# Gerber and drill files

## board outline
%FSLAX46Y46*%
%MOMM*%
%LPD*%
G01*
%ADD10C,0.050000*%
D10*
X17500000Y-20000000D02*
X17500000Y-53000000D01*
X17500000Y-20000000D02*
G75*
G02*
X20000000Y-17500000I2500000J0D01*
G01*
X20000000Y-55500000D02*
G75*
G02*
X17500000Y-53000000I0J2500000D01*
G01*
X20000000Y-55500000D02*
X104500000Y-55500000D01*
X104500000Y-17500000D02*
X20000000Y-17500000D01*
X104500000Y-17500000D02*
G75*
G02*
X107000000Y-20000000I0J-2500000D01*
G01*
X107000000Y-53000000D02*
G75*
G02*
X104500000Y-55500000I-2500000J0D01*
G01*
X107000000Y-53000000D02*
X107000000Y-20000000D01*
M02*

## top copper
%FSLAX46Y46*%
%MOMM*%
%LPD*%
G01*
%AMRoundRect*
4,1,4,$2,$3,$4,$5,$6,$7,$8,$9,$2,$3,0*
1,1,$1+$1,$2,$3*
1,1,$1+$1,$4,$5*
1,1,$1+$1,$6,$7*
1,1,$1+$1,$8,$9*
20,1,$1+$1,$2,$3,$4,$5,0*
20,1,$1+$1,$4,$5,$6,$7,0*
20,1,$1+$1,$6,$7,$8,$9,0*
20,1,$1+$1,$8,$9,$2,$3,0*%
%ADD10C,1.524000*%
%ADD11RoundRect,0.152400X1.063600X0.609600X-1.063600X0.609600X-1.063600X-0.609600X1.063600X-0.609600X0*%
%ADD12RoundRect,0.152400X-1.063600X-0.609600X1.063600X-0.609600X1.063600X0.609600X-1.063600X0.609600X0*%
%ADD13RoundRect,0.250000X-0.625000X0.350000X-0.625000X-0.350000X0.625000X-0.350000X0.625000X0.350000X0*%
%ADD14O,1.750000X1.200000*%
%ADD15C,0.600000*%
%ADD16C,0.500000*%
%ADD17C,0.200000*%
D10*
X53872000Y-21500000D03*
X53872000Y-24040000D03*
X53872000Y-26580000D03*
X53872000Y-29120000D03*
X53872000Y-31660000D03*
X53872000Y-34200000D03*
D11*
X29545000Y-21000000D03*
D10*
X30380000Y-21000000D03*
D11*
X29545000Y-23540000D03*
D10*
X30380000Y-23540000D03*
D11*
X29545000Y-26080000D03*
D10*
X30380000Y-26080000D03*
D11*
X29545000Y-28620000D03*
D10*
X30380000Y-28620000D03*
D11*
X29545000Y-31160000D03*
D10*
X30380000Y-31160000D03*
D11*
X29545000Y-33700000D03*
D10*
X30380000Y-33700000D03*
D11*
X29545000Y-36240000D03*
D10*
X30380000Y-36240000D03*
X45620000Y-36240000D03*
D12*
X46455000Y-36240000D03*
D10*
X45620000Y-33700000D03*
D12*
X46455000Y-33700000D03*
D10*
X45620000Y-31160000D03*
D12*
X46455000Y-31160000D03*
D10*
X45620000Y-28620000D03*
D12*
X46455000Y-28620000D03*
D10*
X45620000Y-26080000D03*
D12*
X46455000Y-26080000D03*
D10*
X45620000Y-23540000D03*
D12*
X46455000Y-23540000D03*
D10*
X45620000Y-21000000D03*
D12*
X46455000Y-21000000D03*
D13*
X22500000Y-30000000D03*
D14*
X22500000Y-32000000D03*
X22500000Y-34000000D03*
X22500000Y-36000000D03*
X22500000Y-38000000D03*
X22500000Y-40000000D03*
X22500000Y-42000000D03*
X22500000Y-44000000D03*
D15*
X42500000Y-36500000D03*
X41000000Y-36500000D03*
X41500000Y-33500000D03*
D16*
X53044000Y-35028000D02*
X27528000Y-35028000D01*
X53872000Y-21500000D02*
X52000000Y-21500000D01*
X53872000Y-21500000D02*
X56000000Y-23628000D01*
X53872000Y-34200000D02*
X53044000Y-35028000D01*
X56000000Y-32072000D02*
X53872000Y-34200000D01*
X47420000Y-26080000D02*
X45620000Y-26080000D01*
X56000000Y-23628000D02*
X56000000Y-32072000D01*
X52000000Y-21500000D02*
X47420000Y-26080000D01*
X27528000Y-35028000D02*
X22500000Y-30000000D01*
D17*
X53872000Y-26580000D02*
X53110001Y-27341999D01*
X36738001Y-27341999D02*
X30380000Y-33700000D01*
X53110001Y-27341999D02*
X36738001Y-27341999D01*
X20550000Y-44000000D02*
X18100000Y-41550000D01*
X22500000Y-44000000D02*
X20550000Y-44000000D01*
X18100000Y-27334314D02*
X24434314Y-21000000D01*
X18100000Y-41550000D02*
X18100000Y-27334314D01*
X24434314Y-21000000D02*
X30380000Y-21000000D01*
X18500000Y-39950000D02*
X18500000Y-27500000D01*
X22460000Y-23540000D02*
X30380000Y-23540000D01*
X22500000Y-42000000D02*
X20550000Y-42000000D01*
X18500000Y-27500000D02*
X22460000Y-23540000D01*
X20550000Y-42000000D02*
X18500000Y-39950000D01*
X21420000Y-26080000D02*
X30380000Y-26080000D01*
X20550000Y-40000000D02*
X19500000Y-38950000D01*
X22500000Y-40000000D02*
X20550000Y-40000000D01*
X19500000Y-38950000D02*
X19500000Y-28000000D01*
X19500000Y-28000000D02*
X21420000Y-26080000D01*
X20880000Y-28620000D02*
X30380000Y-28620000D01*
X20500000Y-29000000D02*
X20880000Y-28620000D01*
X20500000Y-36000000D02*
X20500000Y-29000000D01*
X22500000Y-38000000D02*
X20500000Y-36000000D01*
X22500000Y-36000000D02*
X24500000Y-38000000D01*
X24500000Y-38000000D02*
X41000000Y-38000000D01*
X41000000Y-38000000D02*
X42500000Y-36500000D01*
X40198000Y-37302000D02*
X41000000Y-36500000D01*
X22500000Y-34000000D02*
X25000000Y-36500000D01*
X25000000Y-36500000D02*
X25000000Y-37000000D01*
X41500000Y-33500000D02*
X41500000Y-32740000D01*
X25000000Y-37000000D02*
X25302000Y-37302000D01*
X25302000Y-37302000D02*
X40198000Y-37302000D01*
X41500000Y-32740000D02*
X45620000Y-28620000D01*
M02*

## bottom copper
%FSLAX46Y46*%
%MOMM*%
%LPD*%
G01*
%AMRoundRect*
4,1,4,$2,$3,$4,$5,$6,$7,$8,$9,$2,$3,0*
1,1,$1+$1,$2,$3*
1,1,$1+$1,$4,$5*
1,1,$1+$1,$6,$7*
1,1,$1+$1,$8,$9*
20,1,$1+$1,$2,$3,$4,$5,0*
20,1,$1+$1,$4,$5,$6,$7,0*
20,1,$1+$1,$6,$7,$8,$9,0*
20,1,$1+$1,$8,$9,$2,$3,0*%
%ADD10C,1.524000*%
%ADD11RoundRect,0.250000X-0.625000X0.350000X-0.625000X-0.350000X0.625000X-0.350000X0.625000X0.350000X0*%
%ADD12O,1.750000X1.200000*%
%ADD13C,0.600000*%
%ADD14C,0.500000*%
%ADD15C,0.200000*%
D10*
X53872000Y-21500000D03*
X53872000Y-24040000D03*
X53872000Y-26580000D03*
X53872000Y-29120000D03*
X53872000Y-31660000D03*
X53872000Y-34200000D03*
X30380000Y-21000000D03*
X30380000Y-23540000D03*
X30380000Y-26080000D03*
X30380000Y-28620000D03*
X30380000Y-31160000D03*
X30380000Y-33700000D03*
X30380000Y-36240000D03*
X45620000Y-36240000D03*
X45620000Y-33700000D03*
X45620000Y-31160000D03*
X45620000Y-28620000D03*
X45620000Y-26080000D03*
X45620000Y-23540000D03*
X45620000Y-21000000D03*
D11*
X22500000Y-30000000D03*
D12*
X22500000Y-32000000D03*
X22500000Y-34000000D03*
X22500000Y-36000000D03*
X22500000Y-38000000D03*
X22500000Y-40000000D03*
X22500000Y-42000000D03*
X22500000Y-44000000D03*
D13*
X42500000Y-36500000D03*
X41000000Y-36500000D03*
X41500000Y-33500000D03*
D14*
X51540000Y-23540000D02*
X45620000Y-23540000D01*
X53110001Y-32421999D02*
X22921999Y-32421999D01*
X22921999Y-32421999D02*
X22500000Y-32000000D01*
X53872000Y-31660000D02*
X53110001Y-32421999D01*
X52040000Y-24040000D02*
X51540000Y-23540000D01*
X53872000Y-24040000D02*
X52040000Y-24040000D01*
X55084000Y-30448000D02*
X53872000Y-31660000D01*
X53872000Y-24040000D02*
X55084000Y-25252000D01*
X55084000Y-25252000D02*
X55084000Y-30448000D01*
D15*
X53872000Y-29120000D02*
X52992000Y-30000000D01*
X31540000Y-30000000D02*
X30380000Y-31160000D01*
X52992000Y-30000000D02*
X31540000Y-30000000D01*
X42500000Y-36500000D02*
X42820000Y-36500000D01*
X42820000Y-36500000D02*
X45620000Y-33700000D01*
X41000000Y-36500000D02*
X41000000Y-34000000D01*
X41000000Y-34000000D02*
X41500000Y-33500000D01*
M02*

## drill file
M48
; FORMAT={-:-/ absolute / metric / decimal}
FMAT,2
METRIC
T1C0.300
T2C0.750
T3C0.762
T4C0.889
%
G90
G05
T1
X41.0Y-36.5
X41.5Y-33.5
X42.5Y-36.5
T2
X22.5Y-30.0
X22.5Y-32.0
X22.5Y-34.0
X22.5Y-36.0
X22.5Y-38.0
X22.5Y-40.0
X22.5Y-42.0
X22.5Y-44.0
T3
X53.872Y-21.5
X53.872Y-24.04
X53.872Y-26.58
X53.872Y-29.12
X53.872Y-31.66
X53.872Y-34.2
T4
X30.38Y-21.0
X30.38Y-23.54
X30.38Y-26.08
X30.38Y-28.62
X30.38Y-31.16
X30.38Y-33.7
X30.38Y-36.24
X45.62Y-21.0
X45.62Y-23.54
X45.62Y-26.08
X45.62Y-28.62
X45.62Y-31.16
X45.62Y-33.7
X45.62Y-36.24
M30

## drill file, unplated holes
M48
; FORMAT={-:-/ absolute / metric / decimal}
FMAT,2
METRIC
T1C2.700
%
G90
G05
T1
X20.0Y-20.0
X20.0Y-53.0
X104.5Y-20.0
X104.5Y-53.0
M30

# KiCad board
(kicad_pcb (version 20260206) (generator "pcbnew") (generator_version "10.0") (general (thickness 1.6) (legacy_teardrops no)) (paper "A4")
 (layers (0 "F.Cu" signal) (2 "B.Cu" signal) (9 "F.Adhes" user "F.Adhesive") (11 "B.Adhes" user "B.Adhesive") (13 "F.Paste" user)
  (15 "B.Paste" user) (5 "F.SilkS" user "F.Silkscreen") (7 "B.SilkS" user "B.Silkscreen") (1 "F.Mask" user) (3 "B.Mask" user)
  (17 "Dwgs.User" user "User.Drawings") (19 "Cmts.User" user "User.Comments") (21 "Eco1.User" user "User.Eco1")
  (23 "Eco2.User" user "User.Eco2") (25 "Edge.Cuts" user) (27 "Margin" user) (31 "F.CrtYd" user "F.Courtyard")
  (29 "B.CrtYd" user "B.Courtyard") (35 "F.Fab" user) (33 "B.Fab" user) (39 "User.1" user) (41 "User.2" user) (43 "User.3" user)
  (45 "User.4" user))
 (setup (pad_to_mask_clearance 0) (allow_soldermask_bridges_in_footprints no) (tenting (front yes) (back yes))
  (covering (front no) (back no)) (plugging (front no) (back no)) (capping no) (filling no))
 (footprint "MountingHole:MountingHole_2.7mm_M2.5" (layer "F.Cu") (at 104.5 53)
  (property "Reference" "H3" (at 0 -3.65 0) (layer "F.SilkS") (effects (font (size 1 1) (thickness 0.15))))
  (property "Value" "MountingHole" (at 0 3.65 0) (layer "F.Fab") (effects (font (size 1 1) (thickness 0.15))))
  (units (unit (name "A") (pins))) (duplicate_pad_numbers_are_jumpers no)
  (pad "" np_thru_hole circle (at 0 0) (size 2.7 2.7) (drill 2.7) (layers "*.Cu" "*.Mask")))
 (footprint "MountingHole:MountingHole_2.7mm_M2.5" (layer "F.Cu") (at 20 20)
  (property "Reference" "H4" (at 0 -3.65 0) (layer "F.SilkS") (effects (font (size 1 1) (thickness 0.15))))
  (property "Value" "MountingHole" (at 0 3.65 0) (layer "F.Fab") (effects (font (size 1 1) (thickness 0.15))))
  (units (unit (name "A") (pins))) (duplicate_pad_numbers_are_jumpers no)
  (pad "" np_thru_hole circle (at 0 0) (size 2.7 2.7) (drill 2.7) (layers "*.Cu" "*.Mask")))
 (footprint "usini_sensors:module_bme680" (layer "F.Cu") (at 53.872 34.2)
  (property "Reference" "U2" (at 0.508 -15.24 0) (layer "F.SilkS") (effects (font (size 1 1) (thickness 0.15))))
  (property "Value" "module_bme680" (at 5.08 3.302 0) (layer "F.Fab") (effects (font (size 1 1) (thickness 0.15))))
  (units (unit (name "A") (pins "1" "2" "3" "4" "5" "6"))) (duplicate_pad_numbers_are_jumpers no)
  (pad "1" thru_hole circle (at 0 -12.7) (size 1.524 1.524) (drill 0.762) (layers "*.Cu" "*.Mask") (remove_unused_layers no) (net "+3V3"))
  (pad "2" thru_hole circle (at 0 -10.16) (size 1.524 1.524) (drill 0.762) (layers "*.Cu" "*.Mask") (remove_unused_layers no) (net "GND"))
  (pad "3" thru_hole circle (at 0 -7.62) (size 1.524 1.524) (drill 0.762) (layers "*.Cu" "*.Mask") (remove_unused_layers no) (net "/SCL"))
  (pad "4" thru_hole circle (at 0 -5.08) (size 1.524 1.524) (drill 0.762) (layers "*.Cu" "*.Mask") (remove_unused_layers no) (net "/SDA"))
  (pad "5" thru_hole circle (at 0 -2.54) (size 1.524 1.524) (drill 0.762) (layers "*.Cu" "*.Mask") (remove_unused_layers no) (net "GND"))
  (pad "6" thru_hole circle (at 0 0) (size 1.524 1.524) (drill 0.762) (layers "*.Cu" "*.Mask") (remove_unused_layers no) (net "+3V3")))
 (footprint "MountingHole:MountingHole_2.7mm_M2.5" (layer "F.Cu") (at 104.5 20)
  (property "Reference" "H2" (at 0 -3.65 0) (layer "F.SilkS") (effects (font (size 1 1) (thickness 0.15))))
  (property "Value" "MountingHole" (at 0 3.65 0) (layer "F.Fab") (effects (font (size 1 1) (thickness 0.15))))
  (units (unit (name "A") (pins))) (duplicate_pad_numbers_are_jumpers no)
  (pad "" np_thru_hole circle (at 0 0) (size 2.7 2.7) (drill 2.7) (layers "*.Cu" "*.Mask")))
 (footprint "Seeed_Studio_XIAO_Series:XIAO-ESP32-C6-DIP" (layer "F.Cu") (at 38 28.62 90)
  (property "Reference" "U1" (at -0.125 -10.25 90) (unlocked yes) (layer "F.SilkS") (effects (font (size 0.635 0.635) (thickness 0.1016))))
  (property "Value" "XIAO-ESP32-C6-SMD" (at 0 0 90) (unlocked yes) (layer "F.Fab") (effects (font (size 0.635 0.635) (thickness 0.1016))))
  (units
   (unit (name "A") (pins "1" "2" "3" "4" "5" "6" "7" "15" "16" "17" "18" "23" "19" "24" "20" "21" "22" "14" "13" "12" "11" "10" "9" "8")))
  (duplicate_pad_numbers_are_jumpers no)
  (pad "1" smd roundrect (at 7.62 -8.455 180) (size 2.432 1.524) (layers "F.Cu" "F.Mask") (roundrect_rratio 0.1) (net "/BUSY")
   (thermal_bridge_angle 45))
  (pad "1" thru_hole circle (at 7.62 -7.62 180) (size 1.524 1.524) (drill 0.889) (layers "*.Cu" "*.Mask") (remove_unused_layers no)
   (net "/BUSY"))
  (pad "2" smd roundrect (at 5.08 -8.455 180) (size 2.432 1.524) (layers "F.Cu" "F.Mask") (roundrect_rratio 0.1) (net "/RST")
   (thermal_bridge_angle 45))
  (pad "2" thru_hole circle (at 5.08 -7.62 180) (size 1.524 1.524) (drill 0.889) (layers "*.Cu" "*.Mask") (remove_unused_layers no)
   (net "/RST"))
  (pad "3" smd roundrect (at 2.54 -8.455 180) (size 2.432 1.524) (layers "F.Cu" "F.Mask") (roundrect_rratio 0.1) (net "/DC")
   (thermal_bridge_angle 45))
  (pad "3" thru_hole circle (at 2.54 -7.62 180) (size 1.524 1.524) (drill 0.889) (layers "*.Cu" "*.Mask") (remove_unused_layers no)
   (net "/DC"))
  (pad "4" smd roundrect (at 0 -8.455 180) (size 2.432 1.524) (layers "F.Cu" "F.Mask") (roundrect_rratio 0.1) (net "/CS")
   (thermal_bridge_angle 45))
  (pad "4" thru_hole circle (at 0 -7.62 180) (size 1.524 1.524) (drill 0.889) (layers "*.Cu" "*.Mask") (remove_unused_layers no) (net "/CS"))
  (pad "5" smd roundrect (at -2.54 -8.455 180) (size 2.432 1.524) (layers "F.Cu" "F.Mask") (roundrect_rratio 0.1) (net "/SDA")
   (thermal_bridge_angle 45))
  (pad "5" thru_hole circle (at -2.54 -7.62 180) (size 1.524 1.524) (drill 0.889) (layers "*.Cu" "*.Mask") (remove_unused_layers no)
   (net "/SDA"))
  (pad "6" smd roundrect (at -5.08 -8.455 180) (size 2.432 1.524) (layers "F.Cu" "F.Mask") (roundrect_rratio 0.1) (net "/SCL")
   (thermal_bridge_angle 45))
  (pad "6" thru_hole circle (at -5.08 -7.62 180) (size 1.524 1.524) (drill 0.889) (layers "*.Cu" "*.Mask") (remove_unused_layers no)
   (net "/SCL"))
  (pad "7" smd roundrect (at -7.62 -8.455 180) (size 2.432 1.524) (layers "F.Cu" "F.Mask") (roundrect_rratio 0.1)
   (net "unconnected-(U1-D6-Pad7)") (thermal_bridge_angle 45))
  (pad "7" thru_hole circle (at -7.62 -7.62 180) (size 1.524 1.524) (drill 0.889) (layers "*.Cu" "*.Mask") (remove_unused_layers no)
   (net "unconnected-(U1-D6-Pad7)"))
  (pad "8" thru_hole circle (at -7.62 7.62) (size 1.524 1.524) (drill 0.889) (layers "*.Cu" "*.Mask") (remove_unused_layers no)
   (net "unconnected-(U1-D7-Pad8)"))
  (pad "8" smd roundrect (at -7.62 8.455) (size 2.432 1.524) (layers "F.Cu" "F.Mask") (roundrect_rratio 0.1)
   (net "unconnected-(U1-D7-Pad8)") (thermal_bridge_angle 45))
  (pad "9" thru_hole circle (at -5.08 7.62) (size 1.524 1.524) (drill 0.889) (layers "*.Cu" "*.Mask") (remove_unused_layers no) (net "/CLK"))
  (pad "9" smd roundrect (at -5.08 8.455) (size 2.432 1.524) (layers "F.Cu" "F.Mask") (roundrect_rratio 0.1) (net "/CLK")
   (thermal_bridge_angle 45))
  (pad "10" thru_hole circle (at -2.54 7.62) (size 1.524 1.524) (drill 0.889) (layers "*.Cu" "*.Mask") (remove_unused_layers no)
   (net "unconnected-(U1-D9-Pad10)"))
  (pad "10" smd roundrect (at -2.54 8.455) (size 2.432 1.524) (layers "F.Cu" "F.Mask") (roundrect_rratio 0.1)
   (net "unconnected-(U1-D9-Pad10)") (thermal_bridge_angle 45))
  (pad "11" thru_hole circle (at 0 7.62) (size 1.524 1.524) (drill 0.889) (layers "*.Cu" "*.Mask") (remove_unused_layers no) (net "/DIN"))
  (pad "11" smd roundrect (at 0 8.455) (size 2.432 1.524) (layers "F.Cu" "F.Mask") (roundrect_rratio 0.1) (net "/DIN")
   (thermal_bridge_angle 45))
  (pad "12" thru_hole circle (at 2.54 7.62) (size 1.524 1.524) (drill 0.889) (layers "*.Cu" "*.Mask") (remove_unused_layers no) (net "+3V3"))
  (pad "12" smd roundrect (at 2.54 8.455) (size 2.432 1.524) (layers "F.Cu" "F.Mask") (roundrect_rratio 0.1) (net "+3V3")
   (thermal_bridge_angle 45))
  (pad "13" thru_hole circle (at 5.08 7.62) (size 1.524 1.524) (drill 0.889) (layers "*.Cu" "*.Mask") (remove_unused_layers no) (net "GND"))
  (pad "13" smd roundrect (at 5.08 8.455) (size 2.432 1.524) (layers "F.Cu" "F.Mask") (roundrect_rratio 0.1) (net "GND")
   (thermal_bridge_angle 45))
  (pad "14" thru_hole circle (at 7.62 7.62) (size 1.524 1.524) (drill 0.889) (layers "*.Cu" "*.Mask") (remove_unused_layers no)
   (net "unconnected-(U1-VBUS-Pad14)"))
  (pad "14" smd roundrect (at 7.62 8.455) (size 2.432 1.524) (layers "F.Cu" "F.Mask") (roundrect_rratio 0.1)
   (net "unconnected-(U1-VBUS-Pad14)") (thermal_bridge_angle 45)))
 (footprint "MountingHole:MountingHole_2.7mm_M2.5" (layer "F.Cu") (at 20 53)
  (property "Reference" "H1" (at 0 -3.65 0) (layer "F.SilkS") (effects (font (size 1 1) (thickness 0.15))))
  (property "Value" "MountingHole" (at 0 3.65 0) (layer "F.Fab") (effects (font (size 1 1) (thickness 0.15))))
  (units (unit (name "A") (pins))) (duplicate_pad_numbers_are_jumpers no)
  (pad "" np_thru_hole circle (at 0 0) (size 2.7 2.7) (drill 2.7) (layers "*.Cu" "*.Mask")))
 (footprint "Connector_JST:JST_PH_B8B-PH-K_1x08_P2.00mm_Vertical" (layer "F.Cu") (at 22.5 30 -90)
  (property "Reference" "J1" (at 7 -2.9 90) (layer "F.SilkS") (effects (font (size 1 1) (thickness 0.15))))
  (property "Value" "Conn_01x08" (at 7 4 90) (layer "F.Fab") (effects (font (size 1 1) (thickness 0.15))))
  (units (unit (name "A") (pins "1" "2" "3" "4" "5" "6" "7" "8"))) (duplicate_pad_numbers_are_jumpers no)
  (pad "1" thru_hole roundrect (at 0 0 270) (size 1.2 1.75) (drill 0.75) (layers "*.Cu" "*.Mask") (remove_unused_layers no)
   (roundrect_rratio 0.208333) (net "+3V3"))
  (pad "2" thru_hole oval (at 2 0 270) (size 1.2 1.75) (drill 0.75) (layers "*.Cu" "*.Mask") (remove_unused_layers no) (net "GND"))
  (pad "3" thru_hole oval (at 4 0 270) (size 1.2 1.75) (drill 0.75) (layers "*.Cu" "*.Mask") (remove_unused_layers no) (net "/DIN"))
  (pad "4" thru_hole oval (at 6 0 270) (size 1.2 1.75) (drill 0.75) (layers "*.Cu" "*.Mask") (remove_unused_layers no) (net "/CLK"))
  (pad "5" thru_hole oval (at 8 0 270) (size 1.2 1.75) (drill 0.75) (layers "*.Cu" "*.Mask") (remove_unused_layers no) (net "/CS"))
  (pad "6" thru_hole oval (at 10 0 270) (size 1.2 1.75) (drill 0.75) (layers "*.Cu" "*.Mask") (remove_unused_layers no) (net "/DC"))
  (pad "7" thru_hole oval (at 12 0 270) (size 1.2 1.75) (drill 0.75) (layers "*.Cu" "*.Mask") (remove_unused_layers no) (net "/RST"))
  (pad "8" thru_hole oval (at 14 0 270) (size 1.2 1.75) (drill 0.75) (layers "*.Cu" "*.Mask") (remove_unused_layers no) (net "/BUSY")))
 (gr_line (start 17.5 20) (end 17.5 53) (stroke (width 0.05) (type default)) (layer "Edge.Cuts"))
 (gr_arc (start 17.5 20) (mid 18.232233 18.232233) (end 20 17.5) (stroke (width 0.05) (type default)) (layer "Edge.Cuts"))
 (gr_arc (start 20 55.5) (mid 18.232233 54.767767) (end 17.5 53) (stroke (width 0.05) (type default)) (layer "Edge.Cuts"))
 (gr_line (start 20 55.5) (end 104.5 55.5) (stroke (width 0.05) (type default)) (layer "Edge.Cuts"))
 (gr_line (start 104.5 17.5) (end 20 17.5) (stroke (width 0.05) (type default)) (layer "Edge.Cuts"))
 (gr_arc (start 104.5 17.5) (mid 106.267767 18.232233) (end 107 20) (stroke (width 0.05) (type default)) (layer "Edge.Cuts"))
 (gr_arc (start 107 53) (mid 106.267767 54.767767) (end 104.5 55.5) (stroke (width 0.05) (type default)) (layer "Edge.Cuts"))
 (gr_line (start 107 53) (end 107 20) (stroke (width 0.05) (type default)) (layer "Edge.Cuts"))
 (segment (start 53.044 35.028) (end 27.528 35.028) (width 0.5) (layer "F.Cu") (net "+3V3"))
 (segment (start 53.872 21.5) (end 52 21.5) (width 0.5) (layer "F.Cu") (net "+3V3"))
 (segment (start 53.872 21.5) (end 56 23.628) (width 0.5) (layer "F.Cu") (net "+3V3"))
 (segment (start 53.872 34.2) (end 53.044 35.028) (width 0.5) (layer "F.Cu") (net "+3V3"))
 (segment (start 56 32.072) (end 53.872 34.2) (width 0.5) (layer "F.Cu") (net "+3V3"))
 (segment (start 47.42 26.08) (end 45.62 26.08) (width 0.5) (layer "F.Cu") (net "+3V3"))
 (segment (start 56 23.628) (end 56 32.072) (width 0.5) (layer "F.Cu") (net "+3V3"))
 (segment (start 52 21.5) (end 47.42 26.08) (width 0.5) (layer "F.Cu") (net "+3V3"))
 (segment (start 27.528 35.028) (end 22.5 30) (width 0.5) (layer "F.Cu") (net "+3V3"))
 (segment (start 51.54 23.54) (end 45.62 23.54) (width 0.5) (layer "B.Cu") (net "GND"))
 (segment (start 53.110001 32.421999) (end 22.921999 32.421999) (width 0.5) (layer "B.Cu") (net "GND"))
 (segment (start 22.921999 32.421999) (end 22.5 32) (width 0.5) (layer "B.Cu") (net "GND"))
 (segment (start 53.872 31.66) (end 53.110001 32.421999) (width 0.5) (layer "B.Cu") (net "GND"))
 (segment (start 52.04 24.04) (end 51.54 23.54) (width 0.5) (layer "B.Cu") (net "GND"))
 (segment (start 53.872 24.04) (end 52.04 24.04) (width 0.5) (layer "B.Cu") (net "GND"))
 (segment (start 55.084 30.448) (end 53.872 31.66) (width 0.5) (layer "B.Cu") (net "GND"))
 (segment (start 53.872 24.04) (end 55.084 25.252) (width 0.5) (layer "B.Cu") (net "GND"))
 (segment (start 55.084 25.252) (end 55.084 30.448) (width 0.5) (layer "B.Cu") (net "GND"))
 (segment (start 53.872 26.58) (end 53.110001 27.341999) (width 0.2) (layer "F.Cu") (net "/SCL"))
 (segment (start 36.738001 27.341999) (end 30.38 33.7) (width 0.2) (layer "F.Cu") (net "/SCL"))
 (segment (start 53.110001 27.341999) (end 36.738001 27.341999) (width 0.2) (layer "F.Cu") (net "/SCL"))
 (segment (start 53.872 29.12) (end 52.992 30) (width 0.2) (layer "B.Cu") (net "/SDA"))
 (segment (start 31.54 30) (end 30.38 31.16) (width 0.2) (layer "B.Cu") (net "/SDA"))
 (segment (start 52.992 30) (end 31.54 30) (width 0.2) (layer "B.Cu") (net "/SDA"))
 (segment (start 20.55 44) (end 18.1 41.55) (width 0.2) (layer "F.Cu") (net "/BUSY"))
 (segment (start 22.5 44) (end 20.55 44) (width 0.2) (layer "F.Cu") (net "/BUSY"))
 (segment (start 18.1 27.334314) (end 24.434314 21) (width 0.2) (layer "F.Cu") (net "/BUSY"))
 (segment (start 18.1 41.55) (end 18.1 27.334314) (width 0.2) (layer "F.Cu") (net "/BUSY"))
 (segment (start 24.434314 21) (end 30.38 21) (width 0.2) (layer "F.Cu") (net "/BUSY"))
 (segment (start 18.5 39.95) (end 18.5 27.5) (width 0.2) (layer "F.Cu") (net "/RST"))
 (segment (start 22.46 23.54) (end 30.38 23.54) (width 0.2) (layer "F.Cu") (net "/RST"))
 (segment (start 22.5 42) (end 20.55 42) (width 0.2) (layer "F.Cu") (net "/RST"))
 (segment (start 18.5 27.5) (end 22.46 23.54) (width 0.2) (layer "F.Cu") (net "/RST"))
 (segment (start 20.55 42) (end 18.5 39.95) (width 0.2) (layer "F.Cu") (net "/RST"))
 (segment (start 21.42 26.08) (end 30.38 26.08) (width 0.2) (layer "F.Cu") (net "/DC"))
 (segment (start 20.55 40) (end 19.5 38.95) (width 0.2) (layer "F.Cu") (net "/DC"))
 (segment (start 22.5 40) (end 20.55 40) (width 0.2) (layer "F.Cu") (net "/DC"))
 (segment (start 19.5 38.95) (end 19.5 28) (width 0.2) (layer "F.Cu") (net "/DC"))
 (segment (start 19.5 28) (end 21.42 26.08) (width 0.2) (layer "F.Cu") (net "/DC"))
 (segment (start 20.88 28.62) (end 30.38 28.62) (width 0.2) (layer "F.Cu") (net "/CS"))
 (segment (start 20.5 29) (end 20.88 28.62) (width 0.2) (layer "F.Cu") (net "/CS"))
 (segment (start 20.5 36) (end 20.5 29) (width 0.2) (layer "F.Cu") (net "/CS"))
 (segment (start 22.5 38) (end 20.5 36) (width 0.2) (layer "F.Cu") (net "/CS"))
 (segment (start 22.5 36) (end 24.5 38) (width 0.2) (layer "F.Cu") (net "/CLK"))
 (segment (start 24.5 38) (end 41 38) (width 0.2) (layer "F.Cu") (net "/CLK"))
 (segment (start 41 38) (end 42.5 36.5) (width 0.2) (layer "F.Cu") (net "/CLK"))
 (via (at 42.5 36.5) (size 0.6) (drill 0.3) (layers "F.Cu" "B.Cu") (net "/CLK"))
 (segment (start 42.5 36.5) (end 42.82 36.5) (width 0.2) (layer "B.Cu") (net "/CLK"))
 (segment (start 42.82 36.5) (end 45.62 33.7) (width 0.2) (layer "B.Cu") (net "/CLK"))
 (segment (start 40.198 37.302) (end 41 36.5) (width 0.2) (layer "F.Cu") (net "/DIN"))
 (segment (start 22.5 34) (end 25 36.5) (width 0.2) (layer "F.Cu") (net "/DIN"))
 (segment (start 25 36.5) (end 25 37) (width 0.2) (layer "F.Cu") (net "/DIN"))
 (segment (start 41.5 33.5) (end 41.5 32.74) (width 0.2) (layer "F.Cu") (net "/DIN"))
 (segment (start 25 37) (end 25.302 37.302) (width 0.2) (layer "F.Cu") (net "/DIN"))
 (segment (start 25.302 37.302) (end 40.198 37.302) (width 0.2) (layer "F.Cu") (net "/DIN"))
 (segment (start 41.5 32.74) (end 45.62 28.62) (width 0.2) (layer "F.Cu") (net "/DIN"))
 (via (at 41 36.5) (size 0.6) (drill 0.3) (layers "F.Cu" "B.Cu") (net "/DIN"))
 (via (at 41.5 33.5) (size 0.6) (drill 0.3) (layers "F.Cu" "B.Cu") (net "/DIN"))
 (segment (start 41 36.5) (end 41 34) (width 0.2) (layer "B.Cu") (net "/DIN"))
 (segment (start 41 34) (end 41.5 33.5) (width 0.2) (layer "B.Cu") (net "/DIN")))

